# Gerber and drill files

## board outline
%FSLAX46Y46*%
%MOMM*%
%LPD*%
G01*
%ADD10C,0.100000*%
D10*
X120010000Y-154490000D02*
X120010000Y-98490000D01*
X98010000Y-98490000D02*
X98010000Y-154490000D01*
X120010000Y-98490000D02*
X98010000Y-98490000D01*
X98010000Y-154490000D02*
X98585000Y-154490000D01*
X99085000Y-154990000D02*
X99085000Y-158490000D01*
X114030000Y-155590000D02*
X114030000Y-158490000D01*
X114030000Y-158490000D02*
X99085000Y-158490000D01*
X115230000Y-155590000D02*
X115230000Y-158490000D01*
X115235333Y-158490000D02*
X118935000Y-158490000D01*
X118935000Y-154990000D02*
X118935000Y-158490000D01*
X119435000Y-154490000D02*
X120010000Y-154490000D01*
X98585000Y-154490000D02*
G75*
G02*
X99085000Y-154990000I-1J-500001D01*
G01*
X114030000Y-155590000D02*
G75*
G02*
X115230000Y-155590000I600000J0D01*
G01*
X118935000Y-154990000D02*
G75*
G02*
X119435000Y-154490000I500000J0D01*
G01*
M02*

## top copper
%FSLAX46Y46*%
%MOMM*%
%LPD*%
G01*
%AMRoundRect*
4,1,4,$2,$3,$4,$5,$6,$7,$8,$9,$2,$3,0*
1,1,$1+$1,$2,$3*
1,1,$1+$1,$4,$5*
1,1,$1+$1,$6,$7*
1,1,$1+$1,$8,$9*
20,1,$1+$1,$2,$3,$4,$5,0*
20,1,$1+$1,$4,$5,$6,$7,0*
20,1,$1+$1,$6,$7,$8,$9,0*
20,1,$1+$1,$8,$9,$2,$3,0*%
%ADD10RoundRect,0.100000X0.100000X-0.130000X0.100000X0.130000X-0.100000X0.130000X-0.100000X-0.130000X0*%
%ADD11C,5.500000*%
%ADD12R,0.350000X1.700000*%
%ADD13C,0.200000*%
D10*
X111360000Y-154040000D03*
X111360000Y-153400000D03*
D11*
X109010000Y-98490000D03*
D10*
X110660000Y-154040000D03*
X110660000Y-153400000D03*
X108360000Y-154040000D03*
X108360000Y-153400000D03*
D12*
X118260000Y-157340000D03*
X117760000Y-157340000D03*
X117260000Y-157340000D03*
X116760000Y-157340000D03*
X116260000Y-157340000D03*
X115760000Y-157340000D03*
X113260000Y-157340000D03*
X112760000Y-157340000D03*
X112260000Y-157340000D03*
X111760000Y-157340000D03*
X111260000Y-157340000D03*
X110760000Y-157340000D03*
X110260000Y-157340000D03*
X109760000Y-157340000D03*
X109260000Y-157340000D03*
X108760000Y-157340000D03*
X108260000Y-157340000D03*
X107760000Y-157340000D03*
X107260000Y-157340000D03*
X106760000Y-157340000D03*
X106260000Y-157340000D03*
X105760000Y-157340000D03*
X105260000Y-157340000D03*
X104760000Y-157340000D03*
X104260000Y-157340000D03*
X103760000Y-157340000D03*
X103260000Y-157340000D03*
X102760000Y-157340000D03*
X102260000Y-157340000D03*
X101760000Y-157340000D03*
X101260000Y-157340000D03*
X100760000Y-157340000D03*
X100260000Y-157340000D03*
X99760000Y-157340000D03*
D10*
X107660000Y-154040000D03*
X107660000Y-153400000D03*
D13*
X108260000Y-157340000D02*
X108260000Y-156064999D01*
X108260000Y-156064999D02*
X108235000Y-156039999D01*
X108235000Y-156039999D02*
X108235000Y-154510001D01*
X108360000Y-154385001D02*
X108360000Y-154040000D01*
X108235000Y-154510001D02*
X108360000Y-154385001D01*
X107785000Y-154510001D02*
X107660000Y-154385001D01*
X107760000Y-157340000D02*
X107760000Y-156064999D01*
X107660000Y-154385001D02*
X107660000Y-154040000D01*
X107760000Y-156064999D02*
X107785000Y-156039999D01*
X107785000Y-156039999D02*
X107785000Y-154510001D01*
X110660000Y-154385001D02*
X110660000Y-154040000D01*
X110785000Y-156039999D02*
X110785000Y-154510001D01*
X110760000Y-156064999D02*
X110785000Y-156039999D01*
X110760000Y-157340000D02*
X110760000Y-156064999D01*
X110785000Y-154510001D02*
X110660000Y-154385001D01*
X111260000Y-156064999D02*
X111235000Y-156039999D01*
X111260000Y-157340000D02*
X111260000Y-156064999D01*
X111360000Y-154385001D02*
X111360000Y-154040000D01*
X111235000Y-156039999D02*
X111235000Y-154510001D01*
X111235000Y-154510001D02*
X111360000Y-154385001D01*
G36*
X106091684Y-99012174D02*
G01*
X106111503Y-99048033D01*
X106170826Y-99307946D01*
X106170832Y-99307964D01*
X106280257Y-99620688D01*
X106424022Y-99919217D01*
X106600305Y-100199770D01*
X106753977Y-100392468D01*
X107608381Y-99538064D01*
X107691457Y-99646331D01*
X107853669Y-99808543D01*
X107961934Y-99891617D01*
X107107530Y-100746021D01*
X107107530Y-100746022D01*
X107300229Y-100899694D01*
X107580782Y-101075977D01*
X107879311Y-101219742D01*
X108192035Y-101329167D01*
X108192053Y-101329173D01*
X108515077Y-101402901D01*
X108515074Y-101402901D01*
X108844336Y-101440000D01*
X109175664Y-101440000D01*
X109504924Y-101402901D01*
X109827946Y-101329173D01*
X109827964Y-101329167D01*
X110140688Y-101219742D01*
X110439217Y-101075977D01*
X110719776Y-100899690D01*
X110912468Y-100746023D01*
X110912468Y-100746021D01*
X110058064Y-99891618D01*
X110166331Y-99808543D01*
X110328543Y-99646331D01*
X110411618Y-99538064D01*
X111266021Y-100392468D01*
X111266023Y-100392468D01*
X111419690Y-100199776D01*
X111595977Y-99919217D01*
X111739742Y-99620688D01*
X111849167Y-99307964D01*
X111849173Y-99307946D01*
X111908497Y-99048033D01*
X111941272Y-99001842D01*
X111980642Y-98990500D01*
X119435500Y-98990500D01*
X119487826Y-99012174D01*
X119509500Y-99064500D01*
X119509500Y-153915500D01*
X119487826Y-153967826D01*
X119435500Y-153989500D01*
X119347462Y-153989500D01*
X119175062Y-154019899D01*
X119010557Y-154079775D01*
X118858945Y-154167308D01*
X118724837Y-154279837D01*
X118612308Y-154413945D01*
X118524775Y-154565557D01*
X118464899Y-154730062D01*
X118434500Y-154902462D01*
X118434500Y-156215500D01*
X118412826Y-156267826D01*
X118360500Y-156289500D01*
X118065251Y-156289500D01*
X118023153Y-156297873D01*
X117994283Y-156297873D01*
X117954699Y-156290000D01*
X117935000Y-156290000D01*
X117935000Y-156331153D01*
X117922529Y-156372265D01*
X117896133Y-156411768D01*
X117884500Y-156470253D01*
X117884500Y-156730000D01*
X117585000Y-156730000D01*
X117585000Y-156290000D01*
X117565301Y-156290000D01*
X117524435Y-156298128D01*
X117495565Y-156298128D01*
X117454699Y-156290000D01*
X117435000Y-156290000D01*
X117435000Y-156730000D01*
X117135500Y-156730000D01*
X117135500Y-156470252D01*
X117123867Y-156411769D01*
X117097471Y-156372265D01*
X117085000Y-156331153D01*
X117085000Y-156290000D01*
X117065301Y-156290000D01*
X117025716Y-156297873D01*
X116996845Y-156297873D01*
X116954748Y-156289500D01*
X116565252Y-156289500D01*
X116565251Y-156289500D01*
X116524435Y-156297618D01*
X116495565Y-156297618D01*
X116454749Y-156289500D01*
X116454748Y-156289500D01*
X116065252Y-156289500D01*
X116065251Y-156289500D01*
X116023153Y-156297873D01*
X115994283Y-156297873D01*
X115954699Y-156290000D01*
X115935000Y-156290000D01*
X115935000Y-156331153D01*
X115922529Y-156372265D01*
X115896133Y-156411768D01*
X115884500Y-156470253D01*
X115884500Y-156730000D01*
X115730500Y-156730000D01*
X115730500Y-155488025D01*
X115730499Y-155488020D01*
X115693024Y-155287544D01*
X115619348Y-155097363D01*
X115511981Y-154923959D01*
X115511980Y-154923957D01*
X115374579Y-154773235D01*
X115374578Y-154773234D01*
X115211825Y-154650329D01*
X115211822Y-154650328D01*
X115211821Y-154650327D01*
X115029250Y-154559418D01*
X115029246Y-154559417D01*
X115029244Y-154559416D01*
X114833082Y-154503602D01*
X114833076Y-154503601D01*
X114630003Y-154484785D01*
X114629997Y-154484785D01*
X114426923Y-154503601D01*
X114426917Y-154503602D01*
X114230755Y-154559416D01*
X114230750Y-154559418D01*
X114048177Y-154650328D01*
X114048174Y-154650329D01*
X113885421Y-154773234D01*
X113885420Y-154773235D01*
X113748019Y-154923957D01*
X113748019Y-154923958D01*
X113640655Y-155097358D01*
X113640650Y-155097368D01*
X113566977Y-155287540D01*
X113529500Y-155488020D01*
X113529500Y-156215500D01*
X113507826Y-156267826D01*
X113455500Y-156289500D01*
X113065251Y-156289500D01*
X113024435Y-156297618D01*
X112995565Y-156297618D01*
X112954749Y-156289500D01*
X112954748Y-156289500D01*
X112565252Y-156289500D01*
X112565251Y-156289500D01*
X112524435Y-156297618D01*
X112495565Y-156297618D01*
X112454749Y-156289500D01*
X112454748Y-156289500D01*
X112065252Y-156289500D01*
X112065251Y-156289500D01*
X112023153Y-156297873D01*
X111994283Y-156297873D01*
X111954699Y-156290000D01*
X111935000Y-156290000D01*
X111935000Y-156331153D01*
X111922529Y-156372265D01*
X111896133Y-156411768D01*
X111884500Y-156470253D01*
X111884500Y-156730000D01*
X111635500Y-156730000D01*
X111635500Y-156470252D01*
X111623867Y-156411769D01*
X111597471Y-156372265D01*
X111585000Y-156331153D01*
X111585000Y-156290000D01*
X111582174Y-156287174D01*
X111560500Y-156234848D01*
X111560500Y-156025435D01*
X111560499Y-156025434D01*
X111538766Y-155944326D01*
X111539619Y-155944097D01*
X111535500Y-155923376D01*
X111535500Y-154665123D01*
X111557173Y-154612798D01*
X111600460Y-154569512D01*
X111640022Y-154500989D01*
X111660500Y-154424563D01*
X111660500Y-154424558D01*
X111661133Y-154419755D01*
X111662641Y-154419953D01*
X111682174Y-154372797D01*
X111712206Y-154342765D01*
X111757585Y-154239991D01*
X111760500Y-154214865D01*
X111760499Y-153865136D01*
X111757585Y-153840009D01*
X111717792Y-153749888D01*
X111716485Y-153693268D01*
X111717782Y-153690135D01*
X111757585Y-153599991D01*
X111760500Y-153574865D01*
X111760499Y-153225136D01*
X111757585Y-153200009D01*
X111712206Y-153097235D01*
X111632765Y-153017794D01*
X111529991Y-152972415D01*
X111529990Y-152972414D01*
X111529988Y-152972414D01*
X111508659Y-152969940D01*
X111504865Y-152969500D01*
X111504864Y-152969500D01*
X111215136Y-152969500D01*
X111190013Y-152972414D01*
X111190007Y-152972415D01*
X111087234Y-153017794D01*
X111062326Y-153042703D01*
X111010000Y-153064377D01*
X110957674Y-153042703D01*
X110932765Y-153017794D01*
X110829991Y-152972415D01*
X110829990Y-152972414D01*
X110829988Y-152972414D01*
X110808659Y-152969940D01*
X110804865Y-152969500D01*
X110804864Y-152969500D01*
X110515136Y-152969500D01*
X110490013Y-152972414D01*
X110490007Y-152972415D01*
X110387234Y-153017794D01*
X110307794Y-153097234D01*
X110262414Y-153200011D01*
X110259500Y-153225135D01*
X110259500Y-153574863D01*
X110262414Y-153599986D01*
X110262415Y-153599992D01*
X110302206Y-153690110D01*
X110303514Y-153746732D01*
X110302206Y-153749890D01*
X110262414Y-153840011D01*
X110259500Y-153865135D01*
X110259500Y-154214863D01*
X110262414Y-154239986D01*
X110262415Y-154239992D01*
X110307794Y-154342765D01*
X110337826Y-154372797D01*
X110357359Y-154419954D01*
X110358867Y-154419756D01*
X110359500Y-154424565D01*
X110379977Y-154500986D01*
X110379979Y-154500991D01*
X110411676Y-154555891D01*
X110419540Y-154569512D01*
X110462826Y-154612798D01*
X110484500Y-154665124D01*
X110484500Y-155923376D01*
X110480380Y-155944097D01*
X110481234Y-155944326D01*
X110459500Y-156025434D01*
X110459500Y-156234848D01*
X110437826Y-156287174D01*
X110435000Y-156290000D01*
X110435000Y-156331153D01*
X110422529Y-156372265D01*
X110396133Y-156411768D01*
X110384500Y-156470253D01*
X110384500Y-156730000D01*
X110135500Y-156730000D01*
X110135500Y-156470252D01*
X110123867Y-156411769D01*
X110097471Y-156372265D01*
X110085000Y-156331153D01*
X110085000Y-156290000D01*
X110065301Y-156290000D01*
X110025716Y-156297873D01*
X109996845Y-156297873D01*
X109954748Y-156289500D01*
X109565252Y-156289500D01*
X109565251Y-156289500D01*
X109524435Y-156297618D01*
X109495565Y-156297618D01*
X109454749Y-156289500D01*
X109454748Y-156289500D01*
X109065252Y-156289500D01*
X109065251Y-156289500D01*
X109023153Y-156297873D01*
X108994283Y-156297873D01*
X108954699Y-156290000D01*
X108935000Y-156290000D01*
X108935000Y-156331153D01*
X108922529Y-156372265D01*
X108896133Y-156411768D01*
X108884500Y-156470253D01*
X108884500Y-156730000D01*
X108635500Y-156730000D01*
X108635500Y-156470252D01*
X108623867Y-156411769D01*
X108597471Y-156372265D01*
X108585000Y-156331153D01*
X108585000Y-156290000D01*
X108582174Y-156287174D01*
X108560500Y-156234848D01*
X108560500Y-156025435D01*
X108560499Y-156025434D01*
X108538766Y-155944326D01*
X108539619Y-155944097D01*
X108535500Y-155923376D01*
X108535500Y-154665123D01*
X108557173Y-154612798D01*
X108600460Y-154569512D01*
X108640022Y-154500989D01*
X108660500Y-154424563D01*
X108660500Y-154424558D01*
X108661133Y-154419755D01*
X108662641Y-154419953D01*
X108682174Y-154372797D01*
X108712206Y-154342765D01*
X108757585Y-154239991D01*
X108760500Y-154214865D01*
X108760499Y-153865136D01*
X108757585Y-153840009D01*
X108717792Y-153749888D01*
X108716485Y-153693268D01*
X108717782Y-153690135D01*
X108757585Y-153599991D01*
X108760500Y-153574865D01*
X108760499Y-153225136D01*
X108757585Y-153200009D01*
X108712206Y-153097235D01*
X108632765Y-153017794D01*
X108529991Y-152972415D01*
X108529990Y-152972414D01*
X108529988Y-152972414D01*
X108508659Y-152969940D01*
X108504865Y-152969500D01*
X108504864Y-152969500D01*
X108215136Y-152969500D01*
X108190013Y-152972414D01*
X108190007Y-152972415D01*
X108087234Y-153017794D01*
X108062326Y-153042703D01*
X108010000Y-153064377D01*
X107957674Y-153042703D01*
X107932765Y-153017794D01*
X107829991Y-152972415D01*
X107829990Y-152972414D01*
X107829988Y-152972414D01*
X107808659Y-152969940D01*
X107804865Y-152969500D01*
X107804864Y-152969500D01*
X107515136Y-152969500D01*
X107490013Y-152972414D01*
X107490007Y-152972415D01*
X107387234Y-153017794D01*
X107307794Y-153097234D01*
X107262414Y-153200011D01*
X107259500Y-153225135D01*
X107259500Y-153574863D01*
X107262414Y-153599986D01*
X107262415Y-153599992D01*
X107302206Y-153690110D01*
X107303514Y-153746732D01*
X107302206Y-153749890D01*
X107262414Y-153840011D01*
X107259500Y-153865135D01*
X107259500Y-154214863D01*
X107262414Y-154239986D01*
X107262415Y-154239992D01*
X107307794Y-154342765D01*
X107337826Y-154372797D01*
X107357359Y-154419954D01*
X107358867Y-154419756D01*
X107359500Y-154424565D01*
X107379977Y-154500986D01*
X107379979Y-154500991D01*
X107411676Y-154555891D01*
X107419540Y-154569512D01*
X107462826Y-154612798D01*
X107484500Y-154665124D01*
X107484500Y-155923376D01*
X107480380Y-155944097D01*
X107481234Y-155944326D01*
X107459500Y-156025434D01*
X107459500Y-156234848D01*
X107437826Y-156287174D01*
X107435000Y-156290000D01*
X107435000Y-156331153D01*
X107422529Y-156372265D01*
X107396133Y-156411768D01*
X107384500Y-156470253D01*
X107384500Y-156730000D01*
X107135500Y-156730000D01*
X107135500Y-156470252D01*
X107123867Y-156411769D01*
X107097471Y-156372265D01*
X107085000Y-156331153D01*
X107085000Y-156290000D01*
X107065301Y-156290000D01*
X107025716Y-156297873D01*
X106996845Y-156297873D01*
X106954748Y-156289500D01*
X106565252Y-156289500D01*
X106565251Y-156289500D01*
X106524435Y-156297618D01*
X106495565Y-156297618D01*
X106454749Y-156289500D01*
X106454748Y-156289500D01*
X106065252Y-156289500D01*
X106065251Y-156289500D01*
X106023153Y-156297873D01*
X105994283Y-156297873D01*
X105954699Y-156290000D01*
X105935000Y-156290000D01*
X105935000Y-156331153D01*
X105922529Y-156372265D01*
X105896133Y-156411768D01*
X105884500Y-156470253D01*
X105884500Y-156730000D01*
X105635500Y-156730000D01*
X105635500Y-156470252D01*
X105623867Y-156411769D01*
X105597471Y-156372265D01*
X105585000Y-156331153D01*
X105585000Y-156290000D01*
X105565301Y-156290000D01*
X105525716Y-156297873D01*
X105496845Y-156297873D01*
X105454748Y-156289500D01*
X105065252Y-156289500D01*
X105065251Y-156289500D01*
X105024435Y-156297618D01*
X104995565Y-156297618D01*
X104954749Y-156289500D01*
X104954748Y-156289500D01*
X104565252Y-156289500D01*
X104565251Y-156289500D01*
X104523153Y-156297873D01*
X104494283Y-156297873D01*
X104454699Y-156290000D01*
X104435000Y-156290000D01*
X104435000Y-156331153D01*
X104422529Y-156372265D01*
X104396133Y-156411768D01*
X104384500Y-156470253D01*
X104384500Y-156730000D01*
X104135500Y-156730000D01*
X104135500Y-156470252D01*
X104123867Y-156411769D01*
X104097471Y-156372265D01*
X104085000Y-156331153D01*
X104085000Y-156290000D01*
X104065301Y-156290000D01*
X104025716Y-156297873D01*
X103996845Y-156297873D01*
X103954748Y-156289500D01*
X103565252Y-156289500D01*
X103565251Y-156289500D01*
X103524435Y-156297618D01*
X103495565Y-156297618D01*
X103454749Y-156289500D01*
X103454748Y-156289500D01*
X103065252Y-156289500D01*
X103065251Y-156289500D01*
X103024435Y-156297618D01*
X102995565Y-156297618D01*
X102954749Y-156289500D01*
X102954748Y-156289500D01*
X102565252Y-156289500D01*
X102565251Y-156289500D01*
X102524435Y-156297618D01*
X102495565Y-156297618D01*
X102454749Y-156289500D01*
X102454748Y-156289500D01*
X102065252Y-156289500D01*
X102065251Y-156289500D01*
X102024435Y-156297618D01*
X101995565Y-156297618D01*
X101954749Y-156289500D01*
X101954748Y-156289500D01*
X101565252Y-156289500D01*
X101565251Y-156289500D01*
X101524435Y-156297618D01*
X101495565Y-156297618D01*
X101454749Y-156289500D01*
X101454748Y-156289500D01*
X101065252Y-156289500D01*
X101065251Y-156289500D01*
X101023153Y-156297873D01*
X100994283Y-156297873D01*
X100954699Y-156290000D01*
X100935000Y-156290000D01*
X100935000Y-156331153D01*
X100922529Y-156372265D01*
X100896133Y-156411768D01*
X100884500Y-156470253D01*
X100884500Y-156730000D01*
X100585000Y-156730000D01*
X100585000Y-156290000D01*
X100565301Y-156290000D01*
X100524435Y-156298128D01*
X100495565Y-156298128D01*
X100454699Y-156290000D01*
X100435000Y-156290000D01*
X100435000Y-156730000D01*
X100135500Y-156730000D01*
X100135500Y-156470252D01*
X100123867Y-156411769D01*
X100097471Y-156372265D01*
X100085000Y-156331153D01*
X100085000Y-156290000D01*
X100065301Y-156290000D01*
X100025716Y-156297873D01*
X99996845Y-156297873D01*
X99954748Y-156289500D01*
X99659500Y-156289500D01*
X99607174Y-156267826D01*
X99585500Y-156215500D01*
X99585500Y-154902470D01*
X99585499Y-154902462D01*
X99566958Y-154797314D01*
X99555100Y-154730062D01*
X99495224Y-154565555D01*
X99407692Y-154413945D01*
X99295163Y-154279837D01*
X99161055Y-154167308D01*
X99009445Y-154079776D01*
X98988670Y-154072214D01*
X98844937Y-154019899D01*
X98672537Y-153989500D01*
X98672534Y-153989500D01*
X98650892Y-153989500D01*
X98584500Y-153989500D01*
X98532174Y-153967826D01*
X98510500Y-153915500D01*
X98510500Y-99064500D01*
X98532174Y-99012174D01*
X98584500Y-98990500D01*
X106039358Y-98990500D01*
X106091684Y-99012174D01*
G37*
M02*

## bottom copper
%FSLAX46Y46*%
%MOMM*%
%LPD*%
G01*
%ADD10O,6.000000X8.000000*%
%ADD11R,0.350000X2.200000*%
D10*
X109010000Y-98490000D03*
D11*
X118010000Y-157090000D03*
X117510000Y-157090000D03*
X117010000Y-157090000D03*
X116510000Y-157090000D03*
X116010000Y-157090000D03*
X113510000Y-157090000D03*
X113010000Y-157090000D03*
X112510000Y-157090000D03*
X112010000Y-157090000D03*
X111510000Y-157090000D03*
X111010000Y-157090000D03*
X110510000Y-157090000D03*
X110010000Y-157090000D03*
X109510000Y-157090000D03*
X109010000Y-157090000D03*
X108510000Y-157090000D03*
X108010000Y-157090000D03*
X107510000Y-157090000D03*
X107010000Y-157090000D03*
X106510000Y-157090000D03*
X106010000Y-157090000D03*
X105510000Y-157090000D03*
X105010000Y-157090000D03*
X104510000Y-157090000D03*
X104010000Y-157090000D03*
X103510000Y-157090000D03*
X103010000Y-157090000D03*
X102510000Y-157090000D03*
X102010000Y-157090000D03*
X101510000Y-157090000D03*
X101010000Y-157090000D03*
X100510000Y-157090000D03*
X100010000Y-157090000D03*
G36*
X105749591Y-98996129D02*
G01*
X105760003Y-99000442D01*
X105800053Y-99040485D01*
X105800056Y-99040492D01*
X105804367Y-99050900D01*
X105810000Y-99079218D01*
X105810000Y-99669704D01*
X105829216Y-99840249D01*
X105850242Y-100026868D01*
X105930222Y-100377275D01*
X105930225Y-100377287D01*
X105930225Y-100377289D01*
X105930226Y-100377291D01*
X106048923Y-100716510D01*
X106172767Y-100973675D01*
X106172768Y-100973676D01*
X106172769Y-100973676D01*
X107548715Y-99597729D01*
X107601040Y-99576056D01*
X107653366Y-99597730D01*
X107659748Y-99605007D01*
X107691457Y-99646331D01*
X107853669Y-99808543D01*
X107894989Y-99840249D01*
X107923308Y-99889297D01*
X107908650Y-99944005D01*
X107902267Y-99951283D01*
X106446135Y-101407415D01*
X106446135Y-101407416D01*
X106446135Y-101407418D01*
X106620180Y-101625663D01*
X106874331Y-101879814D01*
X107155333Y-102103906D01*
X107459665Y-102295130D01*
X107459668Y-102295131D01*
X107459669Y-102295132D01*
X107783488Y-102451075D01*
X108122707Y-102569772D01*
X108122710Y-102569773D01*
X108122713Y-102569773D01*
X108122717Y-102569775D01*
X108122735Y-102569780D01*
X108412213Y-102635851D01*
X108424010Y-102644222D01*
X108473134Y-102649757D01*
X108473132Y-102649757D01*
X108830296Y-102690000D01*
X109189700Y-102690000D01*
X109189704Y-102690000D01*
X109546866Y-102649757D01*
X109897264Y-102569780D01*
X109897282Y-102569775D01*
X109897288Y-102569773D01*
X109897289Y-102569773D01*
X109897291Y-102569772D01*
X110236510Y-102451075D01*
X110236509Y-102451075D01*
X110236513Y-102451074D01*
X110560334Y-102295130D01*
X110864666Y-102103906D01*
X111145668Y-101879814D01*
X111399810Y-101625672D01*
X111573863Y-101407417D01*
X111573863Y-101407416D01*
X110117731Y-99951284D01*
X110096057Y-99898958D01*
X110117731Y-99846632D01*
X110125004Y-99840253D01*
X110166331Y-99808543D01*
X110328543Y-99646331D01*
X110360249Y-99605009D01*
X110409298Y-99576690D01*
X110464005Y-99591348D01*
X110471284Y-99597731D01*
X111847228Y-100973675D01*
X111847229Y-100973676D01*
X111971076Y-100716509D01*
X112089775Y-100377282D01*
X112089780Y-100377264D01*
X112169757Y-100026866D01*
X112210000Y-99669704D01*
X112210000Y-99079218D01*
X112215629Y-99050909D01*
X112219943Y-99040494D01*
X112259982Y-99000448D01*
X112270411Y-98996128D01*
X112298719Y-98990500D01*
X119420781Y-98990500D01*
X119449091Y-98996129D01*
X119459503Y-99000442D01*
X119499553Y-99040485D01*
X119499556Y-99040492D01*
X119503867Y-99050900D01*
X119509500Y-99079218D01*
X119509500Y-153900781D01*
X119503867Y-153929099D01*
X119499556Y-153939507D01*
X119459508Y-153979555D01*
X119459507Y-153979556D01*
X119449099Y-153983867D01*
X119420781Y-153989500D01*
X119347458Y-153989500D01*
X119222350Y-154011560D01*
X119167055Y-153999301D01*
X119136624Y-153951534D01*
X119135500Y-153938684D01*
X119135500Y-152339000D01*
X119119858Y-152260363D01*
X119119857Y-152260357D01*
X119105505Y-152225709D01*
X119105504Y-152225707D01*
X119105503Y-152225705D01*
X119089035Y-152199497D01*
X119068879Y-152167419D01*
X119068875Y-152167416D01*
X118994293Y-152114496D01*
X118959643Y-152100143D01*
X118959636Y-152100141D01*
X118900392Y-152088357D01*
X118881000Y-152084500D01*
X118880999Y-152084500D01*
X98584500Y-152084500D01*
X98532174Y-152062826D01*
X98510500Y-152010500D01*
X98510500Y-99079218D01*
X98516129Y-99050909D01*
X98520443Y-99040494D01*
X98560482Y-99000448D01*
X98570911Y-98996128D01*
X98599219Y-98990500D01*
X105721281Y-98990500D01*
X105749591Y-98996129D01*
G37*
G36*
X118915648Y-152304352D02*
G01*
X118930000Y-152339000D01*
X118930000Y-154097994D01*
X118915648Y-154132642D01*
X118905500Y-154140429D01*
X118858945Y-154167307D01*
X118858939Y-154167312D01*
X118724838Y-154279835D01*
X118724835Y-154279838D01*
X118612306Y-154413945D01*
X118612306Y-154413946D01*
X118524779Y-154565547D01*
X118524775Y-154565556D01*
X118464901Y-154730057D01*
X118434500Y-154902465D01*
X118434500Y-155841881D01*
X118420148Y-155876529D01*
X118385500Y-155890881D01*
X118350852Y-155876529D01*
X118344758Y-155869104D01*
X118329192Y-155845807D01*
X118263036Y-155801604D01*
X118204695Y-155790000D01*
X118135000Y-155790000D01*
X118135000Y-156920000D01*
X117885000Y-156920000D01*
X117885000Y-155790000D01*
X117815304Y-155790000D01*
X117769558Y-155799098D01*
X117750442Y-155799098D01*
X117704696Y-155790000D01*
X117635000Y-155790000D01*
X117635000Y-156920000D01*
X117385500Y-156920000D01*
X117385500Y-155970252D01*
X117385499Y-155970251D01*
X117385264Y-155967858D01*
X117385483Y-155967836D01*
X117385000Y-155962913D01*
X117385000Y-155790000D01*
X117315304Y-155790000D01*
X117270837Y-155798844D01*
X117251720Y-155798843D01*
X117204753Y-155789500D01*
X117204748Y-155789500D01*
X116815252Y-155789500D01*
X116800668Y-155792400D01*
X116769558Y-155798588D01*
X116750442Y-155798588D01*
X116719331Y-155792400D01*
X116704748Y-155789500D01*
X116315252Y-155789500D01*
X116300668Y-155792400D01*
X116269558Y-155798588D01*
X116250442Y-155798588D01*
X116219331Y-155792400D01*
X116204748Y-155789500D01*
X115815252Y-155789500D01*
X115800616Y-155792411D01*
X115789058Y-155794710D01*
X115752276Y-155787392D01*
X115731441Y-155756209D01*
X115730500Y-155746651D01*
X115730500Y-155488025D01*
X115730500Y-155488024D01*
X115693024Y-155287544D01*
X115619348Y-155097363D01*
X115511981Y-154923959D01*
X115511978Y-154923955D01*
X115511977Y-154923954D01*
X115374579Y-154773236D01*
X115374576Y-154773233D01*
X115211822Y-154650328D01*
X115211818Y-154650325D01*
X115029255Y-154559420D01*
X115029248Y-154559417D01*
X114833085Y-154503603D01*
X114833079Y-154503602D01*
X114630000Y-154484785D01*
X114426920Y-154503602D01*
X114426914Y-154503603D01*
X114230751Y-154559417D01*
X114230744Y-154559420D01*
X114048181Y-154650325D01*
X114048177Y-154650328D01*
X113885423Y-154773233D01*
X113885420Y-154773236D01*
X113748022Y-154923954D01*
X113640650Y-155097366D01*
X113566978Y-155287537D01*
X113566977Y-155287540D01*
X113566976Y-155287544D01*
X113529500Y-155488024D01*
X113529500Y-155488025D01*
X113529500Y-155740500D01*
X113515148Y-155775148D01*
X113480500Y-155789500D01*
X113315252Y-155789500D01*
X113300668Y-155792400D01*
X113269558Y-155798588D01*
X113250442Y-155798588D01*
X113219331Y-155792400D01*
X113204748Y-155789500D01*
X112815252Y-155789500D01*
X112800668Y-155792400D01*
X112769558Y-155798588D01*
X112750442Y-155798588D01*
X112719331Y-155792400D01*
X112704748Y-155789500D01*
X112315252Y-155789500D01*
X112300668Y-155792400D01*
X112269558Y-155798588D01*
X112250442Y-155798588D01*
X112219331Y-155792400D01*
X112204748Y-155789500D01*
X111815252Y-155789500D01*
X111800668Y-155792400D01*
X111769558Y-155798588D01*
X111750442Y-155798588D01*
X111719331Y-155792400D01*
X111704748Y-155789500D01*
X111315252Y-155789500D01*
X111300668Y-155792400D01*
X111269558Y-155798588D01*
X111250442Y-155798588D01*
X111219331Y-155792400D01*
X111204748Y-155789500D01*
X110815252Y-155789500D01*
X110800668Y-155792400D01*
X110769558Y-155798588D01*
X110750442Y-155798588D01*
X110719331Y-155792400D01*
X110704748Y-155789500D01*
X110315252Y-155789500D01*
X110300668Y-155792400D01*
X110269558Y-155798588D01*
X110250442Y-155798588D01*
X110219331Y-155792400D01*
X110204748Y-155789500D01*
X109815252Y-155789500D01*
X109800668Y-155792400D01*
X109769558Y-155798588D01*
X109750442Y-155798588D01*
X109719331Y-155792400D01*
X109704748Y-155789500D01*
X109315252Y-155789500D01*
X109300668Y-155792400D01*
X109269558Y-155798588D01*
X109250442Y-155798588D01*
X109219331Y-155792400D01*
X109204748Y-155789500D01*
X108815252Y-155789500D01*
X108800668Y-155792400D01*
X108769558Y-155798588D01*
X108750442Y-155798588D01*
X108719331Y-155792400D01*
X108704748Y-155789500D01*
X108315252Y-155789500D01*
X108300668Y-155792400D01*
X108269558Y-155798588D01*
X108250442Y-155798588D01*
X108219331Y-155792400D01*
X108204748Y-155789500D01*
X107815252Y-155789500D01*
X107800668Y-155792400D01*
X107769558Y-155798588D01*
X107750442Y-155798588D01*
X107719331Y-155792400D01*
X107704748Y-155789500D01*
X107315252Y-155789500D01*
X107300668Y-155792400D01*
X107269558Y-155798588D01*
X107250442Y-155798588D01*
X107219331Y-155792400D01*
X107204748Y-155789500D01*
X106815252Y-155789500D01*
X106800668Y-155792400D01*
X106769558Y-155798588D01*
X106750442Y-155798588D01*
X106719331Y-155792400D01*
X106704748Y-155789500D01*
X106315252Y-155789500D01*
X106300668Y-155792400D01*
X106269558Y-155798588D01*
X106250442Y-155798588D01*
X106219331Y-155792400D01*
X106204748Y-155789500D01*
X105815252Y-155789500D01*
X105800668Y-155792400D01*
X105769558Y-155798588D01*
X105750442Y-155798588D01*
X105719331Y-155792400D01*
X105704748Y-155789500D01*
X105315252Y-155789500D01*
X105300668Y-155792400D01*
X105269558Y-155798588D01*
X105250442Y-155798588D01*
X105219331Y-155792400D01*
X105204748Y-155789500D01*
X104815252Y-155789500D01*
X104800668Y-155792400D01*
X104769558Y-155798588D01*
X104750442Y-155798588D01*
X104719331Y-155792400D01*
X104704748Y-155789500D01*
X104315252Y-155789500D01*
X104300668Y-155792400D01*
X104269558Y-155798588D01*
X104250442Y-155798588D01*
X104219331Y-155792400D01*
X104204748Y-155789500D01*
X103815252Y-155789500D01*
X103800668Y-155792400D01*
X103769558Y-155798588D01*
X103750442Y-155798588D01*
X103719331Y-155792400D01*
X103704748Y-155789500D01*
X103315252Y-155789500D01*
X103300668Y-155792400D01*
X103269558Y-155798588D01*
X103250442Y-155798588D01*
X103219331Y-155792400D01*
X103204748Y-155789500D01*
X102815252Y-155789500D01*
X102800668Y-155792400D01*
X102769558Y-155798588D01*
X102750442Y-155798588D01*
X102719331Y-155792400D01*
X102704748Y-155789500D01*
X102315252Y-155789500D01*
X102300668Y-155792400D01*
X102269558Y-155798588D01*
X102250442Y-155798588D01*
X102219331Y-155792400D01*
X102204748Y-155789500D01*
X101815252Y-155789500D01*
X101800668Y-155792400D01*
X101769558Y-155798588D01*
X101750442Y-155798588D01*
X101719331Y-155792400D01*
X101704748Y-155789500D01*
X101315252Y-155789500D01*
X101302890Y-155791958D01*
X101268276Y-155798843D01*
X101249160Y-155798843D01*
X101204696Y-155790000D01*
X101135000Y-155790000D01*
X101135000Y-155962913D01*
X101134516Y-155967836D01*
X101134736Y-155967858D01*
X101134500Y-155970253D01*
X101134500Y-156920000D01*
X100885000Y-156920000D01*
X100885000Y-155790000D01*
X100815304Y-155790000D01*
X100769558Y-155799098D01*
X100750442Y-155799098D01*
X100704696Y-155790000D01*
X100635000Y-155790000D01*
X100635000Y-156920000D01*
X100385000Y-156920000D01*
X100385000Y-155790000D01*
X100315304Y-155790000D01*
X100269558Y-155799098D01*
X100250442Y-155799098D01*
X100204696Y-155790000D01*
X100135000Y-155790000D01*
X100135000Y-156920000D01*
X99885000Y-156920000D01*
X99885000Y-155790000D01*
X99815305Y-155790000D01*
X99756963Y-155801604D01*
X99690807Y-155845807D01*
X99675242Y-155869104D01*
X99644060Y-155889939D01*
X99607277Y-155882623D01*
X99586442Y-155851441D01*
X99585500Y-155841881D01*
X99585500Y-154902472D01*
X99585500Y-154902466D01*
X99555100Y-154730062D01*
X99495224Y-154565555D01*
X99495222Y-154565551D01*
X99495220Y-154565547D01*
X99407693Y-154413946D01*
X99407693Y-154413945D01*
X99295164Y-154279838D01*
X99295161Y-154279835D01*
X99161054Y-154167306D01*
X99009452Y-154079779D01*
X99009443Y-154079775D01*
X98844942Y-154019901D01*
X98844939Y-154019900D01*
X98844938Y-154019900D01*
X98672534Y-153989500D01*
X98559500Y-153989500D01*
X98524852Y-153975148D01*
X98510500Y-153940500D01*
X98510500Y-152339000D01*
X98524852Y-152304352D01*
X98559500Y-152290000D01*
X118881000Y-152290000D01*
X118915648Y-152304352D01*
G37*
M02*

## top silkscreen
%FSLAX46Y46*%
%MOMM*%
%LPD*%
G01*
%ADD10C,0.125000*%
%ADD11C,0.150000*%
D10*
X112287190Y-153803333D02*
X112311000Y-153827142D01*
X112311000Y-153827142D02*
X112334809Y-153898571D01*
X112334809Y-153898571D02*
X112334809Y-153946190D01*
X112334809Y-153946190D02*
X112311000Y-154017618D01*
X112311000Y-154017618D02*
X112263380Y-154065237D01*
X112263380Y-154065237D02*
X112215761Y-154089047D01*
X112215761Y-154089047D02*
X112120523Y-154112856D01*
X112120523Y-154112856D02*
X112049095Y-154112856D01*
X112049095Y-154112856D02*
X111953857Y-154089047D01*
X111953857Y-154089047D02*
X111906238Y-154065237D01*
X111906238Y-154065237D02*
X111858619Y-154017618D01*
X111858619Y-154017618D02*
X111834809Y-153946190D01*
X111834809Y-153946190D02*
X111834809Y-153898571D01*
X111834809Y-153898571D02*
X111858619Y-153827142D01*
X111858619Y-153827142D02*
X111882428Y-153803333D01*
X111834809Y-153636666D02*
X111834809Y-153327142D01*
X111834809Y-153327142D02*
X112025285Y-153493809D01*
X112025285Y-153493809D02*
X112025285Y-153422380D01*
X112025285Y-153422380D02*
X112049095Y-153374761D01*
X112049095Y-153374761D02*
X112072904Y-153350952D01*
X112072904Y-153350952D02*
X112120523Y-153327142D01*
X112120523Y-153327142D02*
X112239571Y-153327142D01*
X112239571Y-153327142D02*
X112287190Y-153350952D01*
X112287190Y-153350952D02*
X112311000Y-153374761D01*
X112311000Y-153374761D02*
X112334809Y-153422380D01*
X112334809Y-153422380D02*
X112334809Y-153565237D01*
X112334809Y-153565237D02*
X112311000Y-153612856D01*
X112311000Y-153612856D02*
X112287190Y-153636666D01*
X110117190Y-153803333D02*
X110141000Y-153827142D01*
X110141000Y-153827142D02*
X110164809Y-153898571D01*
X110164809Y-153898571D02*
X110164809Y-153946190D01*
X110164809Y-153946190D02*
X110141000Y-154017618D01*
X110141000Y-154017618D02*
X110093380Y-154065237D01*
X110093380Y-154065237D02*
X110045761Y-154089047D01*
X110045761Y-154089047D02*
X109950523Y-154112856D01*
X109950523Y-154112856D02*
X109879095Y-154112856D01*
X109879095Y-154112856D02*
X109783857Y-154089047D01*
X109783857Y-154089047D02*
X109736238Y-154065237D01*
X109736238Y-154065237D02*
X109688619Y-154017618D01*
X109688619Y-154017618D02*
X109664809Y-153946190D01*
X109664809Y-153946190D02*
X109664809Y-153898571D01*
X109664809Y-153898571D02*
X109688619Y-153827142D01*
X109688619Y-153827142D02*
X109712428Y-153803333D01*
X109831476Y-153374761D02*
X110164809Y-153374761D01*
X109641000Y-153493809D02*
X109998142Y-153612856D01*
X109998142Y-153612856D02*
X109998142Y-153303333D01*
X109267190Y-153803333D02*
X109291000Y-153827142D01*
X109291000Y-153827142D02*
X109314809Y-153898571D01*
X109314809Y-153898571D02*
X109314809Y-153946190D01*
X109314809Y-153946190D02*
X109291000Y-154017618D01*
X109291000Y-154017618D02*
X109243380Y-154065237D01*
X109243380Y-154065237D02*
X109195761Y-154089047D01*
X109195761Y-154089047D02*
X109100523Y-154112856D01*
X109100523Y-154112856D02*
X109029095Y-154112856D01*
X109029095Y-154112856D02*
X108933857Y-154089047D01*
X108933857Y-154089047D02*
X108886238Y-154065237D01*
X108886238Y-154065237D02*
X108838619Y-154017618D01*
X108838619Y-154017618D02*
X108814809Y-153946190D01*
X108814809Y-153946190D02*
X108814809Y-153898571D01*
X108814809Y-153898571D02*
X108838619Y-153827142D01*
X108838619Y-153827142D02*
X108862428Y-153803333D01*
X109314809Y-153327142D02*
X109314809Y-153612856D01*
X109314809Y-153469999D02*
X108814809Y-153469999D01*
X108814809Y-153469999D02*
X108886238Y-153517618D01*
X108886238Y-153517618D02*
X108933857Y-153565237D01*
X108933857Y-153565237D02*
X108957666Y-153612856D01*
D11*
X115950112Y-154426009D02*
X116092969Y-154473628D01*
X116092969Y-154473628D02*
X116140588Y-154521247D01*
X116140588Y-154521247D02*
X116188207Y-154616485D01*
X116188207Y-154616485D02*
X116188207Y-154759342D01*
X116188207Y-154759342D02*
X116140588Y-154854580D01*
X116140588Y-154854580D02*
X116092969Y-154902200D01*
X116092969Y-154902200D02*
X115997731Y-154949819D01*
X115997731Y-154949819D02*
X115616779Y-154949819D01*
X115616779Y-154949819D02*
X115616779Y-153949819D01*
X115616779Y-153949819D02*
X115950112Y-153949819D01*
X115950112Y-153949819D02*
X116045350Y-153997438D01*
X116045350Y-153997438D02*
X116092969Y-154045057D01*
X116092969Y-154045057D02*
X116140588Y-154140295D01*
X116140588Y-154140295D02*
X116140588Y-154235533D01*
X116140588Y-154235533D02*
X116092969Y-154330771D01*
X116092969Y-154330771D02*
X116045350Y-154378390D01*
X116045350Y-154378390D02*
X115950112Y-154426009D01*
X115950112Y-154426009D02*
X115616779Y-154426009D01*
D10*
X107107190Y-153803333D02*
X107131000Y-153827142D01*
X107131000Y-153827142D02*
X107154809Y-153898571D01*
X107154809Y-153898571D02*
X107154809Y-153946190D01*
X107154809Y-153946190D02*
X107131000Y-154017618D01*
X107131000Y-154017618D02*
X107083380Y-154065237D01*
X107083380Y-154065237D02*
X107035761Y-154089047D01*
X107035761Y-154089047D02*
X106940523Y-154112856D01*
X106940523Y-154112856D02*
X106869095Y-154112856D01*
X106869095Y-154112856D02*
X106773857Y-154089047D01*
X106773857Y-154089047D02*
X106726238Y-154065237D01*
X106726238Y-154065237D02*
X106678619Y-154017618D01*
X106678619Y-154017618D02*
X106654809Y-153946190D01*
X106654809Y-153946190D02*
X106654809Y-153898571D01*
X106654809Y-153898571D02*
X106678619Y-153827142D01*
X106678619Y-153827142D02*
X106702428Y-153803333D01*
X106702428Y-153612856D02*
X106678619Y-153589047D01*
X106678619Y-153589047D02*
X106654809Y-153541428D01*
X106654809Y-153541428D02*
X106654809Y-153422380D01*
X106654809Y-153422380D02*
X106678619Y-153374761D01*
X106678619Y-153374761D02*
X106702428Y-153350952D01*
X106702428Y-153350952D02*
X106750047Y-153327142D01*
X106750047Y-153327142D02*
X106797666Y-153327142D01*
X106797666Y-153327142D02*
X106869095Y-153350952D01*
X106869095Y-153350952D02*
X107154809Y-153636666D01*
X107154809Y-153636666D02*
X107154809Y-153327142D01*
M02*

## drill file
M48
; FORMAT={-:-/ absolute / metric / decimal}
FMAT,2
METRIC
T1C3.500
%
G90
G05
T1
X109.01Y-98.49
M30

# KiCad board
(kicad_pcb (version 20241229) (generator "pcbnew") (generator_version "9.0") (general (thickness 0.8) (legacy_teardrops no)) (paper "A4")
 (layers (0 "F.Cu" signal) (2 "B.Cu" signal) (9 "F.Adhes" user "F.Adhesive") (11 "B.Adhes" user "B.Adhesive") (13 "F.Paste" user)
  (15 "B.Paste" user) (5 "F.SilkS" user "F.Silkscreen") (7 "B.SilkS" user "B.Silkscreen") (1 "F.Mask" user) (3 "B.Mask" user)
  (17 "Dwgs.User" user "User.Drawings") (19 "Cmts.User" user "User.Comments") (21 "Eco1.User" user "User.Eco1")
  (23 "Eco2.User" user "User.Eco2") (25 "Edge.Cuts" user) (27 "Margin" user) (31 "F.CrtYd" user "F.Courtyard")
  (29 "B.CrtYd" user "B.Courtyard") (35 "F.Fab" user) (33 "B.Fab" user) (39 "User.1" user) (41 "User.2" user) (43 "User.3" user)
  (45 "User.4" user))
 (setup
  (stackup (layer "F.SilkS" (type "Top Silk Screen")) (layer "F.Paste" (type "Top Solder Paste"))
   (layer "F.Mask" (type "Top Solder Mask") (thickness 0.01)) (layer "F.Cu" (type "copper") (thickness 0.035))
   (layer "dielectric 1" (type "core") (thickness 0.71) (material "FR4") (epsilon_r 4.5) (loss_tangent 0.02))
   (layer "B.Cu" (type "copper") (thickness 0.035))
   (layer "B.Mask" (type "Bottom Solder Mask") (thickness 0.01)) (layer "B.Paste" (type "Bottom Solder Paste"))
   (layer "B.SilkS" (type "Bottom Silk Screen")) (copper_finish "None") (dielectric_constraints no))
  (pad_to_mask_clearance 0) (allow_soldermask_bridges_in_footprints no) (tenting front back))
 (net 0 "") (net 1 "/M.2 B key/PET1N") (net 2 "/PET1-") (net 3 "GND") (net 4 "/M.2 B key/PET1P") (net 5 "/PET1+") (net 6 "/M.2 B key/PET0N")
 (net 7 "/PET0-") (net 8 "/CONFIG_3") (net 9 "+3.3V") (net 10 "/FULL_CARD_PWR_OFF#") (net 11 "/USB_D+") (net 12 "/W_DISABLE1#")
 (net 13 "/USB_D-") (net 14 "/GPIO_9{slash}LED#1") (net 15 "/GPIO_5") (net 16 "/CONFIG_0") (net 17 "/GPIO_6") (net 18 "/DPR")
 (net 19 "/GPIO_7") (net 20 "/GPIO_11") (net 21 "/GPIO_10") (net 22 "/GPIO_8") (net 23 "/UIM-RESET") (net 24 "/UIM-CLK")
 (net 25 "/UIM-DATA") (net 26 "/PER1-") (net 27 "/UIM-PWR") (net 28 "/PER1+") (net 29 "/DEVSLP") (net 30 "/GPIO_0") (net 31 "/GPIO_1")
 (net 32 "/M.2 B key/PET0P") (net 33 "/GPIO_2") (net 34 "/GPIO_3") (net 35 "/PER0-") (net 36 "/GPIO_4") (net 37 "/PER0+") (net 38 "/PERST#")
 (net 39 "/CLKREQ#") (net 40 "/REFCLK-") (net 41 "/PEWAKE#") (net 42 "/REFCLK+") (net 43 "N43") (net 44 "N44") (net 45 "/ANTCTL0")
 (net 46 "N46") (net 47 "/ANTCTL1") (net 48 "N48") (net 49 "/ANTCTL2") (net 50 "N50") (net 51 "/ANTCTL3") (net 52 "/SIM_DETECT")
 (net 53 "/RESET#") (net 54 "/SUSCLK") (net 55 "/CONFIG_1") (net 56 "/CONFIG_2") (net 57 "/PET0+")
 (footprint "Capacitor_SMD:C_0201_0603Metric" (layer "F.Cu") (at 111.36 153.72 90)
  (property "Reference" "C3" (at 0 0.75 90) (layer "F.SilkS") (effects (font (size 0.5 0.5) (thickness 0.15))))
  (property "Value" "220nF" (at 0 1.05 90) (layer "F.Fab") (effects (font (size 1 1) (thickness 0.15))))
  (pad "" smd roundrect (at -0.345 0 90) (size 0.318 0.36) (layers "F.Paste") (roundrect_rratio 0.25))
  (pad "" smd roundrect (at 0.345 0 90) (size 0.318 0.36) (layers "F.Paste") (roundrect_rratio 0.25))
  (pad "1" smd roundrect (at -0.32 0 90) (size 0.46 0.4) (layers "F.Cu" "F.Mask") (roundrect_rratio 0.25) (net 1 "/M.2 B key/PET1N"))
  (pad "2" smd roundrect (at 0.32 0 90) (size 0.46 0.4) (layers "F.Cu" "F.Mask") (roundrect_rratio 0.25) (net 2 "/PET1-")))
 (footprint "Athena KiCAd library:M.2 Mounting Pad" (layer "F.Cu") (at 109.01 98.49)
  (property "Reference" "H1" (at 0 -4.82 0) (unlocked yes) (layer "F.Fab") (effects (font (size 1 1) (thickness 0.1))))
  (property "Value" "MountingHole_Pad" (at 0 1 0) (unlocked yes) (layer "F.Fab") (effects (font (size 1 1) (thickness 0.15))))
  (pad "1" thru_hole circle (at 0 0) (size 5.5 5.5) (drill 3.5) (layers "*.Cu" "*.Mask") (remove_unused_layers no) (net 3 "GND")
   (padstack (mode front_inner_back)
    (layer "Inner" (shape circle) (size 5.5 5.5) (zone_connect -1))
    (layer "B.Cu" (shape oval) (size 6 8) (thermal_bridge_angle 45) (zone_connect -1)))))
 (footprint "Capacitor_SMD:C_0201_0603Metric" (layer "F.Cu") (at 110.66 153.72 90)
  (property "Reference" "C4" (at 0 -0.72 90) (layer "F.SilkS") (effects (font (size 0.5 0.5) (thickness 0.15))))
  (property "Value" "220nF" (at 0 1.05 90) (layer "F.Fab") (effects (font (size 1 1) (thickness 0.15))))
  (pad "" smd roundrect (at -0.345 0 90) (size 0.318 0.36) (layers "F.Paste") (roundrect_rratio 0.25))
  (pad "" smd roundrect (at 0.345 0 90) (size 0.318 0.36) (layers "F.Paste") (roundrect_rratio 0.25))
  (pad "1" smd roundrect (at -0.32 0 90) (size 0.46 0.4) (layers "F.Cu" "F.Mask") (roundrect_rratio 0.25) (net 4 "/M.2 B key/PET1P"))
  (pad "2" smd roundrect (at 0.32 0 90) (size 0.46 0.4) (layers "F.Cu" "F.Mask") (roundrect_rratio 0.25) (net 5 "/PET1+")))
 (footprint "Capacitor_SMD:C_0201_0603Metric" (layer "F.Cu") (at 108.36 153.72 90)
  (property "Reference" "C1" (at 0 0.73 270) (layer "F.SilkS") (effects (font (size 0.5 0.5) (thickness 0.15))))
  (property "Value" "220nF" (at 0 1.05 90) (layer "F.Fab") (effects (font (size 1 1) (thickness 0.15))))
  (pad "" smd roundrect (at -0.345 0 90) (size 0.318 0.36) (layers "F.Paste") (roundrect_rratio 0.25))
  (pad "" smd roundrect (at 0.345 0 90) (size 0.318 0.36) (layers "F.Paste") (roundrect_rratio 0.25))
  (pad "1" smd roundrect (at -0.32 0 90) (size 0.46 0.4) (layers "F.Cu" "F.Mask") (roundrect_rratio 0.25) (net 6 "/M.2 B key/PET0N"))
  (pad "2" smd roundrect (at 0.32 0 90) (size 0.46 0.4) (layers "F.Cu" "F.Mask") (roundrect_rratio 0.25) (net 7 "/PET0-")))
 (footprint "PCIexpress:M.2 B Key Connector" (layer "F.Cu") (at 109.01 157.38)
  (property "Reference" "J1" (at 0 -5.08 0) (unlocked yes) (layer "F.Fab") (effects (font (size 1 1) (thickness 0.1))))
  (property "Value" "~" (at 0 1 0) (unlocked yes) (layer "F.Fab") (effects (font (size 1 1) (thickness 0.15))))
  (fp_line (start -11 -2.89) (end -10.425 -2.89) (stroke (width 0.1) (type default)) (layer "Edge.Cuts") (net 6))
  (fp_line (start -9.925 -2.39) (end -9.925 1.11) (stroke (width 0.1) (type default)) (layer "Edge.Cuts") (net 6))
  (fp_line (start 5.02 -1.79) (end 5.02 1.11) (stroke (width 0.1) (type default)) (layer "Edge.Cuts") (net 6))
  (fp_line (start 5.02 1.11) (end -9.925 1.11) (stroke (width 0.1) (type default)) (layer "Edge.Cuts") (net 6))
  (fp_line (start 6.22 -1.79) (end 6.22 1.11) (stroke (width 0.1) (type default)) (layer "Edge.Cuts") (net 6))
  (fp_line (start 6.225333 1.11) (end 9.925 1.11) (stroke (width 0.1) (type default)) (layer "Edge.Cuts") (net 6))
  (fp_line (start 9.925 -2.39) (end 9.925 1.11) (stroke (width 0.1) (type default)) (layer "Edge.Cuts") (net 6))
  (fp_line (start 10.425 -2.89) (end 11 -2.89) (stroke (width 0.1) (type default)) (layer "Edge.Cuts") (net 6))
  (fp_arc (start -10.425 -2.89) (mid -10.071447 -2.743553) (end -9.925 -2.39) (stroke (width 0.1) (type default)) (layer "Edge.Cuts")
   (net 6))
  (fp_arc (start 5.02 -1.79) (mid 5.62 -2.39) (end 6.22 -1.79) (stroke (width 0.1) (type default)) (layer "Edge.Cuts") (net 6))
  (fp_arc (start 9.925 -2.39) (mid 10.071447 -2.743553) (end 10.425 -2.89) (stroke (width 0.1) (type default)) (layer "Edge.Cuts") (net 6))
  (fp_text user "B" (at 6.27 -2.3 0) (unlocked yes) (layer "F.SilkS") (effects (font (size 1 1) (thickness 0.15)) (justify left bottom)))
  (pad "1" smd rect (at 9.25 -0.04 180) (size 0.35 1.7) (layers "F.Cu") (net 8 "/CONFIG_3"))
  (pad "2" smd rect (at 9 -0.29 180) (size 0.35 2.2) (layers "B.Cu") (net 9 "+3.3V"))
  (pad "3" smd rect (at 8.75 -0.04 180) (size 0.35 1.7) (layers "F.Cu") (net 3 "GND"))
  (pad "4" smd rect (at 8.5 -0.29 180) (size 0.35 2.2) (layers "B.Cu") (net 9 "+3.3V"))
  (pad "5" smd rect (at 8.25 -0.04 180) (size 0.35 1.7) (layers "F.Cu") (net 3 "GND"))
  (pad "6" smd rect (at 8 -0.29 180) (size 0.35 2.2) (layers "B.Cu") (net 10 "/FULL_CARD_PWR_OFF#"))
  (pad "7" smd rect (at 7.75 -0.04 180) (size 0.35 1.7) (layers "F.Cu") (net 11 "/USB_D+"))
  (pad "8" smd rect (at 7.5 -0.29 180) (size 0.35 2.2) (layers "B.Cu") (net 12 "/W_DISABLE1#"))
  (pad "9" smd rect (at 7.25 -0.04 180) (size 0.35 1.7) (layers "F.Cu") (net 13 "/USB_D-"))
  (pad "10" smd rect (at 7 -0.29 180) (size 0.35 2.2) (layers "B.Cu") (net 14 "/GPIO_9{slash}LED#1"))
  (pad "11" smd rect (at 6.75 -0.04 180) (size 0.35 1.7) (layers "F.Cu") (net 3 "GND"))
  (pad "20" smd rect (at 4.5 -0.29 180) (size 0.35 2.2) (layers "B.Cu") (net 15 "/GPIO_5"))
  (pad "21" smd rect (at 4.25 -0.04 180) (size 0.35 1.7) (layers "F.Cu") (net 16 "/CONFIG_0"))
  (pad "22" smd rect (at 4 -0.29 180) (size 0.35 2.2) (layers "B.Cu") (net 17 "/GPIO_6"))
  (pad "23" smd rect (at 3.75 -0.04 180) (size 0.35 1.7) (layers "F.Cu") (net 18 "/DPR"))
  (pad "24" smd rect (at 3.5 -0.29 180) (size 0.35 2.2) (layers "B.Cu") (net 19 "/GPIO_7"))
  (pad "25" smd rect (at 3.25 -0.04 180) (size 0.35 1.7) (layers "F.Cu") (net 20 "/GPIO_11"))
  (pad "26" smd rect (at 3 -0.29 180) (size 0.35 2.2) (layers "B.Cu") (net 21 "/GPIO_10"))
  (pad "27" smd rect (at 2.75 -0.04 180) (size 0.35 1.7) (layers "F.Cu") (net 3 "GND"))
  (pad "28" smd rect (at 2.5 -0.29 180) (size 0.35 2.2) (layers "B.Cu") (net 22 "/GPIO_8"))
  (pad "29" smd rect (at 2.25 -0.04 180) (size 0.35 1.7) (layers "F.Cu") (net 1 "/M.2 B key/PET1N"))
  (pad "30" smd rect (at 2 -0.29 180) (size 0.35 2.2) (layers "B.Cu") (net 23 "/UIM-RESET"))
  (pad "31" smd rect (at 1.75 -0.04 180) (size 0.35 1.7) (layers "F.Cu") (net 4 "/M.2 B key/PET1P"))
  (pad "32" smd rect (at 1.5 -0.29 180) (size 0.35 2.2) (layers "B.Cu") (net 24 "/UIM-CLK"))
  (pad "33" smd rect (at 1.25 -0.04 180) (size 0.35 1.7) (layers "F.Cu") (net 3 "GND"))
  (pad "34" smd rect (at 1 -0.29 180) (size 0.35 2.2) (layers "B.Cu") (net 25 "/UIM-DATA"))
  (pad "35" smd rect (at 0.75 -0.04 180) (size 0.35 1.7) (layers "F.Cu") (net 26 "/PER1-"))
  (pad "36" smd rect (at 0.5 -0.29 180) (size 0.35 2.2) (layers "B.Cu") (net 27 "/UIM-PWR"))
  (pad "37" smd rect (at 0.25 -0.04 180) (size 0.35 1.7) (layers "F.Cu") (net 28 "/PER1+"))
  (pad "38" smd rect (at 0 -0.29 180) (size 0.35 2.2) (layers "B.Cu") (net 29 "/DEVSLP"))
  (pad "39" smd rect (at -0.25 -0.04 180) (size 0.35 1.7) (layers "F.Cu") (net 3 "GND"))
  (pad "40" smd rect (at -0.5 -0.29 180) (size 0.35 2.2) (layers "B.Cu") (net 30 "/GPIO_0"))
  (pad "41" smd rect (at -0.75 -0.04 180) (size 0.35 1.7) (layers "F.Cu") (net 6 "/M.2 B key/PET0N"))
  (pad "42" smd rect (at -1 -0.29 180) (size 0.35 2.2) (layers "B.Cu") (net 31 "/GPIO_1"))
  (pad "43" smd rect (at -1.25 -0.04 180) (size 0.35 1.7) (layers "F.Cu") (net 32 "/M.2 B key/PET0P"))
  (pad "44" smd rect (at -1.5 -0.29 180) (size 0.35 2.2) (layers "B.Cu") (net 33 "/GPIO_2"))
  (pad "45" smd rect (at -1.75 -0.04 180) (size 0.35 1.7) (layers "F.Cu") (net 3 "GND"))
  (pad "46" smd rect (at -2 -0.29 180) (size 0.35 2.2) (layers "B.Cu") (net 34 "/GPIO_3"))
  (pad "47" smd rect (at -2.25 -0.04 180) (size 0.35 1.7) (layers "F.Cu") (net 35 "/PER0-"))
  (pad "48" smd rect (at -2.5 -0.29 180) (size 0.35 2.2) (layers "B.Cu") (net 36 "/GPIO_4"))
  (pad "49" smd rect (at -2.75 -0.04 180) (size 0.35 1.7) (layers "F.Cu") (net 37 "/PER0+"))
  (pad "50" smd rect (at -3 -0.29 180) (size 0.35 2.2) (layers "B.Cu") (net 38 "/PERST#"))
  (pad "51" smd rect (at -3.25 -0.04 180) (size 0.35 1.7) (layers "F.Cu") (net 3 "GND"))
  (pad "52" smd rect (at -3.5 -0.29 180) (size 0.35 2.2) (layers "B.Cu") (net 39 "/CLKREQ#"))
  (pad "53" smd rect (at -3.75 -0.04 180) (size 0.35 1.7) (layers "F.Cu") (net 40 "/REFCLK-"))
  (pad "54" smd rect (at -4 -0.29 180) (size 0.35 2.2) (layers "B.Cu") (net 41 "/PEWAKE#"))
  (pad "55" smd rect (at -4.25 -0.04 180) (size 0.35 1.7) (layers "F.Cu") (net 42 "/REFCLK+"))
  (pad "56" smd rect (at -4.5 -0.29 180) (size 0.35 2.2) (layers "B.Cu") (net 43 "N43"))
  (pad "57" smd rect (at -4.75 -0.04 180) (size 0.35 1.7) (layers "F.Cu") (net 3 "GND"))
  (pad "58" smd rect (at -5 -0.29 180) (size 0.35 2.2) (layers "B.Cu") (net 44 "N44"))
  (pad "59" smd rect (at -5.25 -0.04 180) (size 0.35 1.7) (layers "F.Cu") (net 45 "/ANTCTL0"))
  (pad "60" smd rect (at -5.5 -0.29 180) (size 0.35 2.2) (layers "B.Cu") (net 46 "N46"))
  (pad "61" smd rect (at -5.75 -0.04 180) (size 0.35 1.7) (layers "F.Cu") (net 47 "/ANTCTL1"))
  (pad "62" smd rect (at -6 -0.29 180) (size 0.35 2.2) (layers "B.Cu") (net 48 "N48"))
  (pad "63" smd rect (at -6.25 -0.04 180) (size 0.35 1.7) (layers "F.Cu") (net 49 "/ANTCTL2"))
  (pad "64" smd rect (at -6.5 -0.29 180) (size 0.35 2.2) (layers "B.Cu") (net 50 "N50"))
  (pad "65" smd rect (at -6.75 -0.04 180) (size 0.35 1.7) (layers "F.Cu") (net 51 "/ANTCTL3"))
  (pad "66" smd rect (at -7 -0.29 180) (size 0.35 2.2) (layers "B.Cu") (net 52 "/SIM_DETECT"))
  (pad "67" smd rect (at -7.25 -0.04 180) (size 0.35 1.7) (layers "F.Cu") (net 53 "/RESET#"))
  (pad "68" smd rect (at -7.5 -0.29 180) (size 0.35 2.2) (layers "B.Cu") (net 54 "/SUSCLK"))
  (pad "69" smd rect (at -7.75 -0.04 180) (size 0.35 1.7) (layers "F.Cu") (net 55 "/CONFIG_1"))
  (pad "70" smd rect (at -8 -0.29 180) (size 0.35 2.2) (layers "B.Cu") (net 9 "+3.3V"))
  (pad "71" smd rect (at -8.25 -0.04 180) (size 0.35 1.7) (layers "F.Cu") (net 3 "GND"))
  (pad "72" smd rect (at -8.5 -0.29 180) (size 0.35 2.2) (layers "B.Cu") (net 9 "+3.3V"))
  (pad "73" smd rect (at -8.75 -0.04 180) (size 0.35 1.7) (layers "F.Cu") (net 3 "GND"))
  (pad "74" smd rect (at -9 -0.29 180) (size 0.35 2.2) (layers "B.Cu") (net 9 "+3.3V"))
  (pad "75" smd rect (at -9.25 -0.04 180) (size 0.35 1.7) (layers "F.Cu") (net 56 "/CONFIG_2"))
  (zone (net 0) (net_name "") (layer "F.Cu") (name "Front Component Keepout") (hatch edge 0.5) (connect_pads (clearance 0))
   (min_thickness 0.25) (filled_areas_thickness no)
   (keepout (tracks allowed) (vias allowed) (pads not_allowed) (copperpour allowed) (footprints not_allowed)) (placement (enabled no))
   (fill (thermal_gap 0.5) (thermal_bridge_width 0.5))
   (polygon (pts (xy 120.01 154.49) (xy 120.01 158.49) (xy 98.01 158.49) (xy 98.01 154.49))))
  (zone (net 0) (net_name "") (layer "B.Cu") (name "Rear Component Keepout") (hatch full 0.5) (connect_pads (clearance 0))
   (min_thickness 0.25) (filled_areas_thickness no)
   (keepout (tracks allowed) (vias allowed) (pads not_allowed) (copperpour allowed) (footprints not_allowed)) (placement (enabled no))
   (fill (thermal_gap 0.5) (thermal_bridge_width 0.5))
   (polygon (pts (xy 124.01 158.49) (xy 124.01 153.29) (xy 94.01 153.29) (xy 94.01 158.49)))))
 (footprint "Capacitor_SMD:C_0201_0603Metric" (layer "F.Cu") (at 107.66 153.72 90)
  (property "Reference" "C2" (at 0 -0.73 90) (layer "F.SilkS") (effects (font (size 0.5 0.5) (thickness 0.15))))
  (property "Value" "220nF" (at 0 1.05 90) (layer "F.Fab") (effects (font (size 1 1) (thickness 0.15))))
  (pad "" smd roundrect (at -0.345 0 90) (size 0.318 0.36) (layers "F.Paste") (roundrect_rratio 0.25))
  (pad "" smd roundrect (at 0.345 0 90) (size 0.318 0.36) (layers "F.Paste") (roundrect_rratio 0.25))
  (pad "1" smd roundrect (at -0.32 0 90) (size 0.46 0.4) (layers "F.Cu" "F.Mask") (roundrect_rratio 0.25) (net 32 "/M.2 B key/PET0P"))
  (pad "2" smd roundrect (at 0.32 0 90) (size 0.46 0.4) (layers "F.Cu" "F.Mask") (roundrect_rratio 0.25) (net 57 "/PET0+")))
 (gr_line (start 120.01 154.49) (end 120.01 98.49) (stroke (width 0.1) (type default)) (layer "Edge.Cuts"))
 (gr_line (start 98.01 98.49) (end 98.01 154.49) (stroke (width 0.1) (type default)) (layer "Edge.Cuts"))
 (gr_line (start 120.01 98.49) (end 98.01 98.49) (stroke (width 0.1) (type default)) (layer "Edge.Cuts"))
 (segment (start 108.26 157.34) (end 108.26 156.064999) (width 0.2) (layer "F.Cu") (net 6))
 (segment (start 108.26 156.064999) (end 108.235 156.039999) (width 0.2) (layer "F.Cu") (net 6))
 (segment (start 108.235 156.039999) (end 108.235 154.510001) (width 0.2) (layer "F.Cu") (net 6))
 (segment (start 108.36 154.385001) (end 108.36 154.04) (width 0.2) (layer "F.Cu") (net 6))
 (segment (start 108.235 154.510001) (end 108.36 154.385001) (width 0.2) (layer "F.Cu") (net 6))
 (segment (start 107.785 154.510001) (end 107.66 154.385001) (width 0.2) (layer "F.Cu") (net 32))
 (segment (start 107.76 157.34) (end 107.76 156.064999) (width 0.2) (layer "F.Cu") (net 32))
 (segment (start 107.66 154.385001) (end 107.66 154.04) (width 0.2) (layer "F.Cu") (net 32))
 (segment (start 107.76 156.064999) (end 107.785 156.039999) (width 0.2) (layer "F.Cu") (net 32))
 (segment (start 107.785 156.039999) (end 107.785 154.510001) (width 0.2) (layer "F.Cu") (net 32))
 (segment (start 110.66 154.385001) (end 110.66 154.04) (width 0.2) (layer "F.Cu") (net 4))
 (segment (start 110.785 156.039999) (end 110.785 154.510001) (width 0.2) (layer "F.Cu") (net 4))
 (segment (start 110.76 156.064999) (end 110.785 156.039999) (width 0.2) (layer "F.Cu") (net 4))
 (segment (start 110.76 157.34) (end 110.76 156.064999) (width 0.2) (layer "F.Cu") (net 4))
 (segment (start 110.785 154.510001) (end 110.66 154.385001) (width 0.2) (layer "F.Cu") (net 4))
 (segment (start 111.26 156.064999) (end 111.235 156.039999) (width 0.2) (layer "F.Cu") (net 1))
 (segment (start 111.26 157.34) (end 111.26 156.064999) (width 0.2) (layer "F.Cu") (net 1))
 (segment (start 111.36 154.385001) (end 111.36 154.04) (width 0.2) (layer "F.Cu") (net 1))
 (segment (start 111.235 156.039999) (end 111.235 154.510001) (width 0.2) (layer "F.Cu") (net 1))
 (segment (start 111.235 154.510001) (end 111.36 154.385001) (width 0.2) (layer "F.Cu") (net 1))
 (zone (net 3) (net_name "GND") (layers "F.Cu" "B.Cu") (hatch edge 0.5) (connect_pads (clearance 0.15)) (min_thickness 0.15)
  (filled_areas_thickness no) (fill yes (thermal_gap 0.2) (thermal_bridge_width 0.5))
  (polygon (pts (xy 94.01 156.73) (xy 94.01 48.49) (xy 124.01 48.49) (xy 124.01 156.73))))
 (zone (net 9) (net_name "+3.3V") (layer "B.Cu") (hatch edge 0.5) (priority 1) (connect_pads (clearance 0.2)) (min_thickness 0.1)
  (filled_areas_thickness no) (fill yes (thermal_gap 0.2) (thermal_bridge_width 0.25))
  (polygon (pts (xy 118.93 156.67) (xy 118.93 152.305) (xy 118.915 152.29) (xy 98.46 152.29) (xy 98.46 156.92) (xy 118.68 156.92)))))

